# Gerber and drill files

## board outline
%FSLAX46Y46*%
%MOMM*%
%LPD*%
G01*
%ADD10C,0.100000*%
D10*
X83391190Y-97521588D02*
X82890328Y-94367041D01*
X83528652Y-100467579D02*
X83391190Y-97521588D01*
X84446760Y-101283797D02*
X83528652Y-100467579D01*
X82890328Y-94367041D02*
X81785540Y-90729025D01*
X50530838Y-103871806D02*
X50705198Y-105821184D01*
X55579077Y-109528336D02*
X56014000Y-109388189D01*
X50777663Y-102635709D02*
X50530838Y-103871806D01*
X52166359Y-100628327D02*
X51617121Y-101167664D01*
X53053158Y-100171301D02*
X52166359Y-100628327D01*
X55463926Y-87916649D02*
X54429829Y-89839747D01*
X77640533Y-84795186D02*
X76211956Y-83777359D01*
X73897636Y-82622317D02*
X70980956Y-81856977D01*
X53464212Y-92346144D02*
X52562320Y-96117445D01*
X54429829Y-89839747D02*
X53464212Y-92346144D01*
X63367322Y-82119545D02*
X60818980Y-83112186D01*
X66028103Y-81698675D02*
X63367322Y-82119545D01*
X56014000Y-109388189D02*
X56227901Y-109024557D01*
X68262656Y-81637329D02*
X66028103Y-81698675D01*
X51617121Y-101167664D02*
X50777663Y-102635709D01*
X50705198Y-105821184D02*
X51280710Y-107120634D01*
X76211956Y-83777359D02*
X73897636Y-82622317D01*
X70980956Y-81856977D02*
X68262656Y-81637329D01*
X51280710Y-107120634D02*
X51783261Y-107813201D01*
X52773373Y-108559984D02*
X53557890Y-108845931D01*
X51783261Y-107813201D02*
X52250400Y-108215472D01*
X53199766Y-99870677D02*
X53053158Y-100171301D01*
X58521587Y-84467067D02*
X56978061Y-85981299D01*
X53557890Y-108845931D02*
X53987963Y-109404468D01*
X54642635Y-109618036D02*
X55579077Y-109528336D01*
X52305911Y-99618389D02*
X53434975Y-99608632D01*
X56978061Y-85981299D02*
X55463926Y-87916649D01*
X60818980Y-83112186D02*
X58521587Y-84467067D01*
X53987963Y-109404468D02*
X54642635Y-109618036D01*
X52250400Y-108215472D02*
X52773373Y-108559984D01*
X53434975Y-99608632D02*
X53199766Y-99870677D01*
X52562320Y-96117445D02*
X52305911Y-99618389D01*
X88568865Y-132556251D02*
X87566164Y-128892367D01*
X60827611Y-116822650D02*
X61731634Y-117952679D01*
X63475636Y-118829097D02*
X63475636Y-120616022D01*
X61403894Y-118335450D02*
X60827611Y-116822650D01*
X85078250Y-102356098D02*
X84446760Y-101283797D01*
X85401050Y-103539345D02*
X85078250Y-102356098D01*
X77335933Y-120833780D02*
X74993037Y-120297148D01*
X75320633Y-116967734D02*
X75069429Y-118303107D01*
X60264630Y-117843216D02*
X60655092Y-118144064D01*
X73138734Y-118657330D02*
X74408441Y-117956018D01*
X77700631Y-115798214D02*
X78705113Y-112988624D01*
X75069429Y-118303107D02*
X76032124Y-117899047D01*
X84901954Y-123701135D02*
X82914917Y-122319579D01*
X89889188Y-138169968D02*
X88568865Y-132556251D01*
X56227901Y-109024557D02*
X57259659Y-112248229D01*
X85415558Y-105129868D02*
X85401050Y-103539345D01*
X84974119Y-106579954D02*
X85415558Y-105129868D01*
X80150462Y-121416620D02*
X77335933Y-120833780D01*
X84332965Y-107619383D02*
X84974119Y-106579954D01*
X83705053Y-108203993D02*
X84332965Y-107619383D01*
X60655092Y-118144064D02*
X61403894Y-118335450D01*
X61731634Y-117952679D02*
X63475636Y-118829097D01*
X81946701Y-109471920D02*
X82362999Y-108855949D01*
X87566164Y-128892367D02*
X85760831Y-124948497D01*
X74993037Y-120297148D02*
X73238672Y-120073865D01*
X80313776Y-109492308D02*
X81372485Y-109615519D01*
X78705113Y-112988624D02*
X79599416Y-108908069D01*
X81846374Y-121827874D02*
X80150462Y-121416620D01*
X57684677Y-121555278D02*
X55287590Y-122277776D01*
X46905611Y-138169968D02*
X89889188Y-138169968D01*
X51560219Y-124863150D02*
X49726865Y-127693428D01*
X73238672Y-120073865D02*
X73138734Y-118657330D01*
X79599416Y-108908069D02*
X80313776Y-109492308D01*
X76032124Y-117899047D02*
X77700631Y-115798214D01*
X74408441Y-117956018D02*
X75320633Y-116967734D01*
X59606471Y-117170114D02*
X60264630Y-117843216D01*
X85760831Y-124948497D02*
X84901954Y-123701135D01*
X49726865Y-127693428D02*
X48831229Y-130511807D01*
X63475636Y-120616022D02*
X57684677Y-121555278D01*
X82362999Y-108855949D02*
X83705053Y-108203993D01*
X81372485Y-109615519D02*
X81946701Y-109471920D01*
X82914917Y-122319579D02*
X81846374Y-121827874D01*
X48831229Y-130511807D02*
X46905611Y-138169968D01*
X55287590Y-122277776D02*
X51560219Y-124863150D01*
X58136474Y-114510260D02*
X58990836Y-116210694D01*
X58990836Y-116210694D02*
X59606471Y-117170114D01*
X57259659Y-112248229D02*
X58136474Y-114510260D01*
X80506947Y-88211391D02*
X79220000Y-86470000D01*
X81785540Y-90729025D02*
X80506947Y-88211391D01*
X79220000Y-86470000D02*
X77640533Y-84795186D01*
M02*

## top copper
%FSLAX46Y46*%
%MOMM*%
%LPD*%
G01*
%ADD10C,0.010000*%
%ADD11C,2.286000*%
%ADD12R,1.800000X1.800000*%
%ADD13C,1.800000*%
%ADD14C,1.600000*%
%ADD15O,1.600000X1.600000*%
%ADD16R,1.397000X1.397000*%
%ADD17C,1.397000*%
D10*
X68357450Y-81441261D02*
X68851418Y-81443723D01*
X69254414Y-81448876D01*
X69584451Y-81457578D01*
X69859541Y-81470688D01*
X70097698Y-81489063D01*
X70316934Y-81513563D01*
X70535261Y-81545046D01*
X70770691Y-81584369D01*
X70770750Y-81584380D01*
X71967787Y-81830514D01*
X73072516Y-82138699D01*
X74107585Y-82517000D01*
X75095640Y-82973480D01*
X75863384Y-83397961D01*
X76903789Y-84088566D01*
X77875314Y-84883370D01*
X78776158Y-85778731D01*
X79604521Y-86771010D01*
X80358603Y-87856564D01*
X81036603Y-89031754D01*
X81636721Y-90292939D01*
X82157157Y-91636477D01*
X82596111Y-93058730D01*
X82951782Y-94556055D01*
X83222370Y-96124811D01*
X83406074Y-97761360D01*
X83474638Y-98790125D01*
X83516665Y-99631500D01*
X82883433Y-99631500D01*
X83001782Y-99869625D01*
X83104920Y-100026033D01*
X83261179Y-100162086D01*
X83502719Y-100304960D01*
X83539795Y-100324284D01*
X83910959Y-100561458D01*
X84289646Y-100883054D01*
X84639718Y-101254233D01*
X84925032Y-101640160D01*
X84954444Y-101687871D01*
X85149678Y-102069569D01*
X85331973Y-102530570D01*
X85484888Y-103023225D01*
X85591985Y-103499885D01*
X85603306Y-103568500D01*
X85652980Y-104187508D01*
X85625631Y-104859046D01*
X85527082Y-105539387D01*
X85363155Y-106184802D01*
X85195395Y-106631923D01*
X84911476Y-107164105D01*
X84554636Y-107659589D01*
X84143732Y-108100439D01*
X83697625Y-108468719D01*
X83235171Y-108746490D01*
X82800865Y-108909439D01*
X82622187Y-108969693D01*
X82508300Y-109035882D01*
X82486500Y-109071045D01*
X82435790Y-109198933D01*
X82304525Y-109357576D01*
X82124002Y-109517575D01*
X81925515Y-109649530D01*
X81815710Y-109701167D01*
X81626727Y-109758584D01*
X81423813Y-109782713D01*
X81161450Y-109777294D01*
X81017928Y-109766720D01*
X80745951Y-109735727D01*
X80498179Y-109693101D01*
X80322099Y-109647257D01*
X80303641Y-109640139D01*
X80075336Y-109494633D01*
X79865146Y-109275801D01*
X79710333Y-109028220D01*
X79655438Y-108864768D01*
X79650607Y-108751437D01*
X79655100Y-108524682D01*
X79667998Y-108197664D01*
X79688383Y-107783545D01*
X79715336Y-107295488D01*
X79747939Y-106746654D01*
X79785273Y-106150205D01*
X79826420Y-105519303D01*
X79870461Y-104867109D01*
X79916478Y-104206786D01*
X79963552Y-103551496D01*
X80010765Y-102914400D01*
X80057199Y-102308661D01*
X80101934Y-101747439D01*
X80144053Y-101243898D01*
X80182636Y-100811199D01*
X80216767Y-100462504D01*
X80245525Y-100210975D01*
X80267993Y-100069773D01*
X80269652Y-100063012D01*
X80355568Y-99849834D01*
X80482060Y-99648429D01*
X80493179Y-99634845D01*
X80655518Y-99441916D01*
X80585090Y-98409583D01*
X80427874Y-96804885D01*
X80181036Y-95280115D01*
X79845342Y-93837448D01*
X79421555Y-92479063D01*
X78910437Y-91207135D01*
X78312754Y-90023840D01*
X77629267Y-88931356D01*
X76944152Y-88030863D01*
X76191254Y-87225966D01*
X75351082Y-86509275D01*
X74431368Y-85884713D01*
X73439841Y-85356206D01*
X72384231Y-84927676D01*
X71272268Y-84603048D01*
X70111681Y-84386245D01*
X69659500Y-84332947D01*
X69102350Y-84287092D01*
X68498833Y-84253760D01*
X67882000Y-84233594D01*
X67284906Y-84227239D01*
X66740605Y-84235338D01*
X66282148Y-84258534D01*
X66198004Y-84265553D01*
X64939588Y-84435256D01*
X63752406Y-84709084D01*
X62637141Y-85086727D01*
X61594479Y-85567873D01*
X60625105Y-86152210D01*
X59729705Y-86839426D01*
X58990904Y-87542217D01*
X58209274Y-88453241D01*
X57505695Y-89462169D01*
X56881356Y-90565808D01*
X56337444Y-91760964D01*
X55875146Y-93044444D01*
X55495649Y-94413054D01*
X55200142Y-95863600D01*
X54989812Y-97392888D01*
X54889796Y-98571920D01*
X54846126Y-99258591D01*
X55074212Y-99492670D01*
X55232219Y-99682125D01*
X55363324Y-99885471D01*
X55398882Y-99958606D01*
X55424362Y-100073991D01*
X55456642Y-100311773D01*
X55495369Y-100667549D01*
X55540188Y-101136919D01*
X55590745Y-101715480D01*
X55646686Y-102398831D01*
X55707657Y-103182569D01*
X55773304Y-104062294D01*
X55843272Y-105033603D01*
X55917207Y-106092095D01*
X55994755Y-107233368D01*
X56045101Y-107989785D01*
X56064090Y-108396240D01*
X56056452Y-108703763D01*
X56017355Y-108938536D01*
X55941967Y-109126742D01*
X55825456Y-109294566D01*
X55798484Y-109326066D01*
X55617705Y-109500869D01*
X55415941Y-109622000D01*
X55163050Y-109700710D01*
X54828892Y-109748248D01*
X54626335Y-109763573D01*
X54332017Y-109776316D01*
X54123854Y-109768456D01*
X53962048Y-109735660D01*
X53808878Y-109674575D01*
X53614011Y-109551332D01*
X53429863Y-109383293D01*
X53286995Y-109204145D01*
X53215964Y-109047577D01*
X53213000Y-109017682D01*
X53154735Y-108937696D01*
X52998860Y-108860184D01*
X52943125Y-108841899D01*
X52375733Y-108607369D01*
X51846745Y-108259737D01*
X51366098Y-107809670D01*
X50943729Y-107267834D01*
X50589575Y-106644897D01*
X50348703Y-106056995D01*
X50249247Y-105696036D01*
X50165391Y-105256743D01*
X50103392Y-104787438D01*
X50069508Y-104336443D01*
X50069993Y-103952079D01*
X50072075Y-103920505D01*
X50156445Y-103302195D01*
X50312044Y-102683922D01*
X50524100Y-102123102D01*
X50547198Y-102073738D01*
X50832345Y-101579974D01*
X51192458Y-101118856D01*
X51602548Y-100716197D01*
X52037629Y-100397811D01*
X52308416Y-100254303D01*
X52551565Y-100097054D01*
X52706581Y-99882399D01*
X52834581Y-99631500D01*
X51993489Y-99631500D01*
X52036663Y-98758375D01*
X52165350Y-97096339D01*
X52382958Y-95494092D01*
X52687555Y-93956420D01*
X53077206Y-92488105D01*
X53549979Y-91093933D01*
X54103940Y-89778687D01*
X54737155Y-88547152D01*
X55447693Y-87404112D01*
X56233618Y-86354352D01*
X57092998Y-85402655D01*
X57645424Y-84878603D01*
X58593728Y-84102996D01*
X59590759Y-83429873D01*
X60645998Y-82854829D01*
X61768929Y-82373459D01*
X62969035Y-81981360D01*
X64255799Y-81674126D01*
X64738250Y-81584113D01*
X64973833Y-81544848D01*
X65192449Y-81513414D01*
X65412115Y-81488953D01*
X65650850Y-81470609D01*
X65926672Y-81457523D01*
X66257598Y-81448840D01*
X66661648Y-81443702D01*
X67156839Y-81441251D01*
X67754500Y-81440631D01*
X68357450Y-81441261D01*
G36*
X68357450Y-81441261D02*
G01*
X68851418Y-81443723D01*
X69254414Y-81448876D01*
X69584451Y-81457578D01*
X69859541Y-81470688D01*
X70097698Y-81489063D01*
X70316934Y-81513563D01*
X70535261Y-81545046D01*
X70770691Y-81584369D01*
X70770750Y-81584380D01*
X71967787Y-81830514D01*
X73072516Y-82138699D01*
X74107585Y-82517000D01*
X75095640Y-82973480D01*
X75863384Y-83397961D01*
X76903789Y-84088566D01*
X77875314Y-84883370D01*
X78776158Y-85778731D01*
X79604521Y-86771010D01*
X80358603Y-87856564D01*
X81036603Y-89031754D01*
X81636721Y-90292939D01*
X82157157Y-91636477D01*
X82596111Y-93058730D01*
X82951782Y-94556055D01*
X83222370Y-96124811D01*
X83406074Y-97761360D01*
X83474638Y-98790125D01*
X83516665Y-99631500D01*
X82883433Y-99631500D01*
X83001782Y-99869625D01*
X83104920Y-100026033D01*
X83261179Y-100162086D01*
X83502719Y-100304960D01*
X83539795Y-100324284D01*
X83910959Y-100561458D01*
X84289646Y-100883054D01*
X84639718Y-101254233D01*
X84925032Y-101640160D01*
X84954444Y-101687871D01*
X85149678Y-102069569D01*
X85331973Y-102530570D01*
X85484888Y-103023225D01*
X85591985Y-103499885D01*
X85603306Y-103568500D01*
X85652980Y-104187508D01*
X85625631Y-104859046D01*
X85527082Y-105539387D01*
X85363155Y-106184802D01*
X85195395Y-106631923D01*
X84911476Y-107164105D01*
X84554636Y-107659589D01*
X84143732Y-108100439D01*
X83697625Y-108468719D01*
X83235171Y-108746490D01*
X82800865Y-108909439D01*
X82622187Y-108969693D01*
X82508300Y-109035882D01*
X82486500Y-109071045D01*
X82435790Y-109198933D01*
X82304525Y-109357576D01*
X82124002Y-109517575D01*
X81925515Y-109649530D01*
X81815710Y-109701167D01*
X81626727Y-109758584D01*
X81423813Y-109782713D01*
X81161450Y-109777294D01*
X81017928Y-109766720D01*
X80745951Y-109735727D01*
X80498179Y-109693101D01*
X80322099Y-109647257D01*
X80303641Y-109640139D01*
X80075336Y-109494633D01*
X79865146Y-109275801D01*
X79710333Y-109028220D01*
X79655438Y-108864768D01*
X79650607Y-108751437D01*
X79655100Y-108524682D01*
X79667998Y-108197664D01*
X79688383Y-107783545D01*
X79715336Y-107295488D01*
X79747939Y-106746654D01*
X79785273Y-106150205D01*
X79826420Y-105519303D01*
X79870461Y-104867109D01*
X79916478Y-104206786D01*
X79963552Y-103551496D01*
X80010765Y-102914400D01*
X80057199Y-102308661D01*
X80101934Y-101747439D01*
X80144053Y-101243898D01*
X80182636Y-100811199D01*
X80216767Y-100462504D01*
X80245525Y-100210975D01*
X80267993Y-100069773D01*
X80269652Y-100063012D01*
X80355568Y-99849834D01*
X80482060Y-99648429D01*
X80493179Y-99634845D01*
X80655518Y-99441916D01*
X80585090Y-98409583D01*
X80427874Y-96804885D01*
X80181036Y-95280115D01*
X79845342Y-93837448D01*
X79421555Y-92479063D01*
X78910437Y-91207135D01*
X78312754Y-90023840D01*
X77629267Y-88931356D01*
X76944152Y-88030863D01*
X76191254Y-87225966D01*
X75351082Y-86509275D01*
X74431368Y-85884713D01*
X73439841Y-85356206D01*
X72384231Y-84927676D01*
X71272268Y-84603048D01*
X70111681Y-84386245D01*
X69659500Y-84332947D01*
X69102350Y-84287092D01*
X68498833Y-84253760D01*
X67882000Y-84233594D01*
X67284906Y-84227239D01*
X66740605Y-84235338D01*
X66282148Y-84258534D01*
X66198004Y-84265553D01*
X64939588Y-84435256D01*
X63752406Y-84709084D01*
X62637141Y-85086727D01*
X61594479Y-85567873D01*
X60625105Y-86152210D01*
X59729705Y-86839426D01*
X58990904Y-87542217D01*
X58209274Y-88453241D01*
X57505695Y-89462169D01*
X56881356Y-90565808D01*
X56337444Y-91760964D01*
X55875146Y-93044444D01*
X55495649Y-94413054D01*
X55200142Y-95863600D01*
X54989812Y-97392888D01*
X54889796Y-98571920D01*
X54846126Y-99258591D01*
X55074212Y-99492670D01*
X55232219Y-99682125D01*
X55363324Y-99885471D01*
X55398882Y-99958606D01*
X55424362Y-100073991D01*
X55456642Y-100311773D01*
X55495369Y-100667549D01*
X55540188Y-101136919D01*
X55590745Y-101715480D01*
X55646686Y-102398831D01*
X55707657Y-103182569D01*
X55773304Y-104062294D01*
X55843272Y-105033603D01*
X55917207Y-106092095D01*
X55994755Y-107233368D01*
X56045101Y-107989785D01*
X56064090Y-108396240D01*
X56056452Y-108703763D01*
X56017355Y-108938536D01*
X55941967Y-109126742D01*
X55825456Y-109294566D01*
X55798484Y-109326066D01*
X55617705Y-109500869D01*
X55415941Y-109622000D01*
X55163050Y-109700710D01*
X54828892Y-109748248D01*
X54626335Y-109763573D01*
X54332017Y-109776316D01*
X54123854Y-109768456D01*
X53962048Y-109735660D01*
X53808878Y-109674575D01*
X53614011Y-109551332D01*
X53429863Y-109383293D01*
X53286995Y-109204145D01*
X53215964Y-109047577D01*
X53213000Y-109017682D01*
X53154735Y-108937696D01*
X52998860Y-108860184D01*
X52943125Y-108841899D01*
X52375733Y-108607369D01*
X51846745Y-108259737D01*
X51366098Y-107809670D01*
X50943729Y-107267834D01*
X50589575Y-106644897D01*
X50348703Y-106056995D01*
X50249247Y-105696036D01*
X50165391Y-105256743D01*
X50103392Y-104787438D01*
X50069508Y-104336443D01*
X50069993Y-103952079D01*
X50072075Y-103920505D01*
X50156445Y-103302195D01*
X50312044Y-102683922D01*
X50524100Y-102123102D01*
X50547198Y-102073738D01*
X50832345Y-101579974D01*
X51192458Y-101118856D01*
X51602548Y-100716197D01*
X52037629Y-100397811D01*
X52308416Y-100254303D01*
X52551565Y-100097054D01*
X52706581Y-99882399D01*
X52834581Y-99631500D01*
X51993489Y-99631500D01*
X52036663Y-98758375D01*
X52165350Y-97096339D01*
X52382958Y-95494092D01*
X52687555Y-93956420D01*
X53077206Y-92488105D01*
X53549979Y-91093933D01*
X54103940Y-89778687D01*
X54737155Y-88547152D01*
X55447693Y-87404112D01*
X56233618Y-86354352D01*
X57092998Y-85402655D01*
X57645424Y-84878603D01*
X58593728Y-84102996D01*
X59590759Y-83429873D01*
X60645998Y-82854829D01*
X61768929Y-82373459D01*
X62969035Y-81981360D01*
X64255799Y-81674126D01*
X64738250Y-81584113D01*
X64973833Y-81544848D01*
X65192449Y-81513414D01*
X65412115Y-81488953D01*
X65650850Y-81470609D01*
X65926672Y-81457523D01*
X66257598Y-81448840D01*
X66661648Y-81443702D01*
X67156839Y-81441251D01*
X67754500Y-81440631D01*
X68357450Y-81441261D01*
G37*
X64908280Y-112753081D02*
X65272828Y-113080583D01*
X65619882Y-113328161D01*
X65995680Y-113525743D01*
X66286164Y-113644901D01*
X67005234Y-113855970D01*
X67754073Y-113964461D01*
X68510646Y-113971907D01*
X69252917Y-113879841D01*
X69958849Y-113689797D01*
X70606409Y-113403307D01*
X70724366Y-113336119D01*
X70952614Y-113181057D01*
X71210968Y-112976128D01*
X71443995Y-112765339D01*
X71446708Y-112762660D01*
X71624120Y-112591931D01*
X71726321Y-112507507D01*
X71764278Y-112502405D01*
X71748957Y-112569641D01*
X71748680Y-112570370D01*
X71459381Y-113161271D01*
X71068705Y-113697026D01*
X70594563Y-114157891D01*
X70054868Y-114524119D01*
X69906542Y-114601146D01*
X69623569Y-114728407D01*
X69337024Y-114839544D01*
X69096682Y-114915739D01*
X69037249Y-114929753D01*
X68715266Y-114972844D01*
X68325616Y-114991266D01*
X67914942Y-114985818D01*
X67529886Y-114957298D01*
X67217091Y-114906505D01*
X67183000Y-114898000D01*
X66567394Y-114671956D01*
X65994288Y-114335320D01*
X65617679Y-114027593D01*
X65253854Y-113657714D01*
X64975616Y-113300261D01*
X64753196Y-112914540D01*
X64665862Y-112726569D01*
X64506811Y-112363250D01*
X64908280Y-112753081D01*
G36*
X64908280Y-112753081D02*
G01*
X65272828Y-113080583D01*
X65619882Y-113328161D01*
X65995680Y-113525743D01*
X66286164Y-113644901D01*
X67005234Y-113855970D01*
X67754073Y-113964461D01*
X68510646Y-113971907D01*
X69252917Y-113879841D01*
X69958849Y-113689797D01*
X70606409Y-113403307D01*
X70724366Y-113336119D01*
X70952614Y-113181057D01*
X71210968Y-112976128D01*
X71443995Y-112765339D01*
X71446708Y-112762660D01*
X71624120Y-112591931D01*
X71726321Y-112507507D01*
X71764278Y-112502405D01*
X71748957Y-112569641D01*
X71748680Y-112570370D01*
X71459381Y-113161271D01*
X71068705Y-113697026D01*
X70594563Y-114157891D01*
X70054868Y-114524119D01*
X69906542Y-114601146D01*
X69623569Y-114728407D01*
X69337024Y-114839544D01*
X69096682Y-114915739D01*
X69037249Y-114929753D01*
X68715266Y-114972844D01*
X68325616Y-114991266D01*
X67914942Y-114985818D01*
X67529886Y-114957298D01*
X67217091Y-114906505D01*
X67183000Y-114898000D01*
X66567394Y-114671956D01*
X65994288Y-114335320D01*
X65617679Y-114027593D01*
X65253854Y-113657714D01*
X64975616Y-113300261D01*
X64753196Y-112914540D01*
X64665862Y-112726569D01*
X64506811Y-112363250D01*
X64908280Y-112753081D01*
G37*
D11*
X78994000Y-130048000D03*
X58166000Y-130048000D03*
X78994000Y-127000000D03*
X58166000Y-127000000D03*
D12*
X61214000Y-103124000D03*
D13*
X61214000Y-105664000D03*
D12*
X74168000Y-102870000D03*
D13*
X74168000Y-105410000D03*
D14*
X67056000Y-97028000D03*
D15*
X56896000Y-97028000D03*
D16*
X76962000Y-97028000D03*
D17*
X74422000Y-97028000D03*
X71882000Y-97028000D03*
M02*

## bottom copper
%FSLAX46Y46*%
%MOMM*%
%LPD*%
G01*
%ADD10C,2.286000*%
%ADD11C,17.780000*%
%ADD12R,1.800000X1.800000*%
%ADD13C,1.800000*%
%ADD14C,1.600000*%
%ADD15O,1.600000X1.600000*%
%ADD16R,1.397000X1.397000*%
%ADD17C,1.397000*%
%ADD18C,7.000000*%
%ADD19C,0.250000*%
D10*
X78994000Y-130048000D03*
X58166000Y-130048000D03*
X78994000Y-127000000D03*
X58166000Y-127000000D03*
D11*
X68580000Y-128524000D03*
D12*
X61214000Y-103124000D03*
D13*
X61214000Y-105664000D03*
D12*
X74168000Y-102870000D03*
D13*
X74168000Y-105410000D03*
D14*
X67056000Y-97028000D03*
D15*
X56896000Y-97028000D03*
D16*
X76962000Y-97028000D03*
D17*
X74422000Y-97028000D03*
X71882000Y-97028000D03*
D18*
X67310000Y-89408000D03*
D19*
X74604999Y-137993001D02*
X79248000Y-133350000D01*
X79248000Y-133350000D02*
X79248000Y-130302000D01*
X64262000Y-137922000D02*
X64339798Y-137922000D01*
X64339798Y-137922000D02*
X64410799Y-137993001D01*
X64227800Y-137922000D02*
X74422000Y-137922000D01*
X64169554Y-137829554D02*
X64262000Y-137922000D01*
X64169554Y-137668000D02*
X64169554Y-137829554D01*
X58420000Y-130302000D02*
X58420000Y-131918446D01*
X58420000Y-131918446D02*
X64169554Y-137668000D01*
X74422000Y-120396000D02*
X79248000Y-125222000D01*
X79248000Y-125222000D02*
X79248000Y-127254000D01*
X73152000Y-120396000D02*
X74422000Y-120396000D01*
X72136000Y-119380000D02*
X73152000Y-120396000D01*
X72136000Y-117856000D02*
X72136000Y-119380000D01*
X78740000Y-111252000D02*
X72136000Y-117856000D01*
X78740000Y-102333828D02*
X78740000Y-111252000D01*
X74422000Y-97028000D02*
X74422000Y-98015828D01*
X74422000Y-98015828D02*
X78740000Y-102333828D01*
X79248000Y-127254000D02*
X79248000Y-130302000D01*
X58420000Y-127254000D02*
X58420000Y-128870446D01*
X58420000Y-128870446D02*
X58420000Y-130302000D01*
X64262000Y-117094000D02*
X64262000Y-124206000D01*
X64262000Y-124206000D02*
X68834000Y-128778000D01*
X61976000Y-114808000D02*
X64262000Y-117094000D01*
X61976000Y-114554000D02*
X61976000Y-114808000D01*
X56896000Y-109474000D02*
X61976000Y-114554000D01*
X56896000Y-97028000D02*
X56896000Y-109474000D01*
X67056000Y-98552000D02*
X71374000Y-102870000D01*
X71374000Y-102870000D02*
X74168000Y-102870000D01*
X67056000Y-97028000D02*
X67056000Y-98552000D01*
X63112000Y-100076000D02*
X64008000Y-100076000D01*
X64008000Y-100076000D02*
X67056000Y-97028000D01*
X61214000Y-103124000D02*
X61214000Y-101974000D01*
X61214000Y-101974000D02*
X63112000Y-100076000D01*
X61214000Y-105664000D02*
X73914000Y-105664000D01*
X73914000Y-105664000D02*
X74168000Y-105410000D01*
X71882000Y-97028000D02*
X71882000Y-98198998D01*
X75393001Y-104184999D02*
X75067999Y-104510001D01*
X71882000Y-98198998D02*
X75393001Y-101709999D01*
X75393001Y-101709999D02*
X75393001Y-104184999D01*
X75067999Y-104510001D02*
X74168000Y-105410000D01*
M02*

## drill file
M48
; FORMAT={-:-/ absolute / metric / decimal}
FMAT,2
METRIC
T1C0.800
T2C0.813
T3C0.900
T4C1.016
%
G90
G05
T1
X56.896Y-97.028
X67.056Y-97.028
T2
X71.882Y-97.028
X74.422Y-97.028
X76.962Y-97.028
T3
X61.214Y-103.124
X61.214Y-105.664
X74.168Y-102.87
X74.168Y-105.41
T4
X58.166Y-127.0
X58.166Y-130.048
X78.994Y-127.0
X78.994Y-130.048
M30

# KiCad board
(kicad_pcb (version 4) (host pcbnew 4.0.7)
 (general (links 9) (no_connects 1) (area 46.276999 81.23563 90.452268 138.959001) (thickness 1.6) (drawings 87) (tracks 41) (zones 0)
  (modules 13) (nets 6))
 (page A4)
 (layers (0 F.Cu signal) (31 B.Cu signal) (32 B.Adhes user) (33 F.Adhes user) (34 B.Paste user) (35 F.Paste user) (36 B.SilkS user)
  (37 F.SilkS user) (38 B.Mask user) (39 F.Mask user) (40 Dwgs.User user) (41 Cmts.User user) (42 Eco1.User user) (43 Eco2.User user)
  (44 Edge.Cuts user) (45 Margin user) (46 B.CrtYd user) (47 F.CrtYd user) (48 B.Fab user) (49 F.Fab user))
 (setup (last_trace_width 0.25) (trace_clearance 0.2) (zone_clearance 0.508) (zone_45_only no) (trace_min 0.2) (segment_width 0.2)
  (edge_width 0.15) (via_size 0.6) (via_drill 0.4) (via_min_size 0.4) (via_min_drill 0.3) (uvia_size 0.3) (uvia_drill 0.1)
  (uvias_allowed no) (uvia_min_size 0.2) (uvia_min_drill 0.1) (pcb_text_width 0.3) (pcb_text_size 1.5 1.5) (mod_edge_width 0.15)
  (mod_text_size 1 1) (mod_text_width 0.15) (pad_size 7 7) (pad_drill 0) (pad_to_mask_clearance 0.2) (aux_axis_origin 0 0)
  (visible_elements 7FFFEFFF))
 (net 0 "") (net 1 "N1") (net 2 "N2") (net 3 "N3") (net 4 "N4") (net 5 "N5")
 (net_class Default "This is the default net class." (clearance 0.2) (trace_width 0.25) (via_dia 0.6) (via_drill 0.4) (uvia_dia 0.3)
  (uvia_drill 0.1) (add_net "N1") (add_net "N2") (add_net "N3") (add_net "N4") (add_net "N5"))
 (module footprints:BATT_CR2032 (layer B.Cu) (at 68.58 128.524 180)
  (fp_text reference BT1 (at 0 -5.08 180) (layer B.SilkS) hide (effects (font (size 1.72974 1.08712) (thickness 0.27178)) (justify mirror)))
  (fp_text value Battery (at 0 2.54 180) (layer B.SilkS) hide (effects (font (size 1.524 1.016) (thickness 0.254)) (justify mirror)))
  (pad 1 thru_hole circle (at -10.414 -1.524 180) (size 2.286 2.286) (drill 1.016) (layers *.Cu *.Mask B.SilkS) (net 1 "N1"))
  (pad 1 thru_hole circle (at 10.414 -1.524 180) (size 2.286 2.286) (drill 1.016) (layers *.Cu *.Mask B.SilkS) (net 1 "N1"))
  (pad 1 thru_hole circle (at -10.414 1.524 180) (size 2.286 2.286) (drill 1.016) (layers *.Cu *.Mask B.SilkS) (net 1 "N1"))
  (pad 1 thru_hole circle (at 10.414 1.524 180) (size 2.286 2.286) (drill 1.016) (layers *.Cu *.Mask B.SilkS) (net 1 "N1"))
  (pad 2 smd circle (at 0 0 180) (size 17.78 17.78) (layers B.Cu B.Paste B.Mask) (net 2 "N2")))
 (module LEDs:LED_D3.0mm (layer F.Cu) (at 61.214 103.124 270)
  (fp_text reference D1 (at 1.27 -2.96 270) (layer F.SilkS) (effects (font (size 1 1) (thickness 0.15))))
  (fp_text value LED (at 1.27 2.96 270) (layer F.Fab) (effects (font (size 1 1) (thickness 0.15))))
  (pad 1 thru_hole rect (at 0 0 270) (size 1.8 1.8) (drill 0.9) (layers *.Cu *.Mask) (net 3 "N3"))
  (pad 2 thru_hole circle (at 2.54 0 270) (size 1.8 1.8) (drill 0.9) (layers *.Cu *.Mask) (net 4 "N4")))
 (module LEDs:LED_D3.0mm (layer F.Cu) (at 74.168 102.87 270)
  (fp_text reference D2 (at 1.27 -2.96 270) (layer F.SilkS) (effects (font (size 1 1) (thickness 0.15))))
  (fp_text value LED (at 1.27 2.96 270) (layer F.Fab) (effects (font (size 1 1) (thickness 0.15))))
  (pad 1 thru_hole rect (at 0 0 270) (size 1.8 1.8) (drill 0.9) (layers *.Cu *.Mask) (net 3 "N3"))
  (pad 2 thru_hole circle (at 2.54 0 270) (size 1.8 1.8) (drill 0.9) (layers *.Cu *.Mask) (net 4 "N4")))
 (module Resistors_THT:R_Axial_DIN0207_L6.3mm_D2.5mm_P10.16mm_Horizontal (layer B.Cu) (at 67.056 97.028 180)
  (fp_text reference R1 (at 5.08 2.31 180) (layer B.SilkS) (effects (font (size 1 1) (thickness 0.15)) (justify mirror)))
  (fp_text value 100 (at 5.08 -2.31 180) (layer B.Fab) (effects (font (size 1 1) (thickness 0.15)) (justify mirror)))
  (pad 1 thru_hole circle (at 0 0 180) (size 1.6 1.6) (drill 0.8) (layers *.Cu *.Mask) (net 3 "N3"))
  (pad 2 thru_hole oval (at 10.16 0 180) (size 1.6 1.6) (drill 0.8) (layers *.Cu *.Mask) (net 2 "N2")))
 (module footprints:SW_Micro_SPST (layer B.Cu) (at 74.422 97.028 180)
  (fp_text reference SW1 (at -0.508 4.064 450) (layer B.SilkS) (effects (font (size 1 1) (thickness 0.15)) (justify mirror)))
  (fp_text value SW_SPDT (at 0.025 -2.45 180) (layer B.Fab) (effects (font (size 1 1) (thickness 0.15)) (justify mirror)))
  (pad 1 thru_hole rect (at -2.54 0 180) (size 1.397 1.397) (drill 0.8128) (layers *.Cu *.Mask B.SilkS) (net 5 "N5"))
  (pad 2 thru_hole circle (at 0 0 180) (size 1.397 1.397) (drill 0.8128) (layers *.Cu *.Mask B.SilkS) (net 1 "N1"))
  (pad 3 thru_hole circle (at 2.54 0 180) (size 1.397 1.397) (drill 0.8128) (layers *.Cu *.Mask B.SilkS) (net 4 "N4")))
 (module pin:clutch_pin (layer F.Cu) (at 67.31 89.408)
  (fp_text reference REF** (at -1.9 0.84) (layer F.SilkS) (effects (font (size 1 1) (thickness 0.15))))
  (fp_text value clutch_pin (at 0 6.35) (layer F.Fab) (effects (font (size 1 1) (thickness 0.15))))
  (pad 1 smd circle (at 0 0 90) (size 7 7) (layers B.Cu B.Paste B.SilkS B.Mask)))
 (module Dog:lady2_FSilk (layer F.Cu) (at 68.326 109.728)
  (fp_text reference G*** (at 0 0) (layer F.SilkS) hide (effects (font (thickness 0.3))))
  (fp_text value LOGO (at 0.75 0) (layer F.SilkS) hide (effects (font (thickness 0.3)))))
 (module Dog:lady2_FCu (layer F.Cu) (at 67.818 97.536)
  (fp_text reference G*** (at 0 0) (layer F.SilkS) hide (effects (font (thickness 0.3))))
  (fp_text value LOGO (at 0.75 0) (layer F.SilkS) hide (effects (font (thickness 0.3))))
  (fp_poly
   (pts (xy 0.53945 -16.094739) (xy 1.033418 -16.092277) (xy 1.436414 -16.087124) (xy 1.766451 -16.078422) (xy 2.041541 -16.065312)
    (xy 2.279698 -16.046937) (xy 2.498934 -16.022437) (xy 2.717261 -15.990954) (xy 2.952691 -15.951631) (xy 2.95275 -15.95162)
    (xy 4.149787 -15.705486) (xy 5.254516 -15.397301) (xy 6.289585 -15.019) (xy 7.27764 -14.56252) (xy 8.045384 -14.138039)
    (xy 9.085789 -13.447434) (xy 10.057314 -12.65263) (xy 10.958158 -11.757269) (xy 11.786521 -10.76499) (xy 12.540603 -9.679436)
    (xy 13.218603 -8.504246) (xy 13.818721 -7.243061) (xy 14.339157 -5.899523) (xy 14.778111 -4.47727) (xy 15.133782 -2.979945)
    (xy 15.40437 -1.411189) (xy 15.588074 0.22536) (xy 15.656638 1.254125) (xy 15.698665 2.0955) (xy 15.065433 2.0955)
    (xy 15.183782 2.333625) (xy 15.28692 2.490033) (xy 15.443179 2.626086) (xy 15.684719 2.76896) (xy 15.721795 2.788284)
    (xy 16.092959 3.025458) (xy 16.471646 3.347054) (xy 16.821718 3.718233) (xy 17.107032 4.10416) (xy 17.136444 4.151871)
    (xy 17.331678 4.533569) (xy 17.513973 4.99457) (xy 17.666888 5.487225) (xy 17.773985 5.963885) (xy 17.785306 6.0325)
    (xy 17.83498 6.651508) (xy 17.807631 7.323046) (xy 17.709082 8.003387) (xy 17.545155 8.648802) (xy 17.377395 9.095923)
    (xy 17.093476 9.628105) (xy 16.736636 10.123589) (xy 16.325732 10.564439) (xy 15.879625 10.932719) (xy 15.417171 11.21049)
    (xy 14.982865 11.373439) (xy 14.804187 11.433693) (xy 14.6903 11.499882) (xy 14.6685 11.535045) (xy 14.61779 11.662933)
    (xy 14.486525 11.821576) (xy 14.306002 11.981575) (xy 14.107515 12.11353) (xy 13.99771 12.165167) (xy 13.808727 12.222584)
    (xy 13.605813 12.246713) (xy 13.34345 12.241294) (xy 13.199928 12.23072) (xy 12.927951 12.199727) (xy 12.680179 12.157101)
    (xy 12.504099 12.111257) (xy 12.485641 12.104139) (xy 12.257336 11.958633) (xy 12.047146 11.739801) (xy 11.892333 11.49222)
    (xy 11.837438 11.328768) (xy 11.832607 11.215437) (xy 11.8371 10.988682) (xy 11.849998 10.661664) (xy 11.870383 10.247545)
    (xy 11.897336 9.759488) (xy 11.929939 9.210654) (xy 11.967273 8.614205) (xy 12.00842 7.983303) (xy 12.052461 7.331109)
    (xy 12.098478 6.670786) (xy 12.145552 6.015496) (xy 12.192765 5.3784) (xy 12.239199 4.772661) (xy 12.283934 4.211439)
    (xy 12.326053 3.707898) (xy 12.364636 3.275199) (xy 12.398767 2.926504) (xy 12.427525 2.674975) (xy 12.449993 2.533773)
    (xy 12.451652 2.527012) (xy 12.537568 2.313834) (xy 12.66406 2.112429) (xy 12.675179 2.098845) (xy 12.837518 1.905916)
    (xy 12.76709 0.873583) (xy 12.609874 -0.731115) (xy 12.363036 -2.255885) (xy 12.027342 -3.698552) (xy 11.603555 -5.056937)
    (xy 11.092437 -6.328865) (xy 10.494754 -7.51216) (xy 9.811267 -8.604644) (xy 9.126152 -9.505137) (xy 8.373254 -10.310034)
    (xy 7.533082 -11.026725) (xy 6.613368 -11.651287) (xy 5.621841 -12.179794) (xy 4.566231 -12.608324) (xy 3.454268 -12.932952)
    (xy 2.293681 -13.149755) (xy 1.8415 -13.203053) (xy 1.28435 -13.248908) (xy 0.680833 -13.28224) (xy 0.064 -13.302406)
    (xy -0.533094 -13.308761) (xy -1.077395 -13.300662) (xy -1.535852 -13.277466) (xy -1.619996 -13.270447) (xy -2.878412 -13.100744)
    (xy -4.065594 -12.826916) (xy -5.180859 -12.449273) (xy -6.223521 -11.968127) (xy -7.192895 -11.38379) (xy -8.088295 -10.696574)
    (xy -8.827096 -9.993783) (xy -9.608726 -9.082759) (xy -10.312305 -8.073831) (xy -10.936644 -6.970192) (xy -11.480556 -5.775036)
    (xy -11.942854 -4.491556) (xy -12.322351 -3.122946) (xy -12.617858 -1.6724) (xy -12.828188 -0.143112) (xy -12.928204 1.03592)
    (xy -12.971874 1.722591) (xy -12.743788 1.95667) (xy -12.585781 2.146125) (xy -12.454676 2.349471) (xy -12.419118 2.422606)
    (xy -12.393638 2.537991) (xy -12.361358 2.775773) (xy -12.322631 3.131549) (xy -12.277812 3.600919) (xy -12.227255 4.17948)
    (xy -12.171314 4.862831) (xy -12.110343 5.646569) (xy -12.044696 6.526294) (xy -11.974728 7.497603) (xy -11.900793 8.556095)
    (xy -11.823245 9.697368) (xy -11.772899 10.453785) (xy -11.75391 10.86024) (xy -11.761548 11.167763) (xy -11.800645 11.402536)
    (xy -11.876033 11.590742) (xy -11.992544 11.758566) (xy -12.019516 11.790066) (xy -12.200295 11.964869) (xy -12.402059 12.086)
    (xy -12.65495 12.16471) (xy -12.989108 12.212248) (xy -13.191665 12.227573) (xy -13.485983 12.240316) (xy -13.694146 12.232456)
    (xy -13.855952 12.19966) (xy -14.009122 12.138575) (xy -14.203989 12.015332) (xy -14.388137 11.847293) (xy -14.531005 11.668145)
    (xy -14.602036 11.511577) (xy -14.605 11.481682) (xy -14.663265 11.401696) (xy -14.81914 11.324184) (xy -14.874875 11.305899)
    (xy -15.442267 11.071369) (xy -15.971255 10.723737) (xy -16.451902 10.27367) (xy -16.874271 9.731834) (xy -17.228425 9.108897)
    (xy -17.469297 8.520995) (xy -17.568753 8.160036) (xy -17.652609 7.720743) (xy -17.714608 7.251438) (xy -17.748492 6.800443)
    (xy -17.748007 6.416079) (xy -17.745925 6.384505) (xy -17.661555 5.766195) (xy -17.505956 5.147922) (xy -17.2939 4.587102)
    (xy -17.270802 4.537738) (xy -16.985655 4.043974) (xy -16.625542 3.582856) (xy -16.215452 3.180197) (xy -15.780371 2.861811)
    (xy -15.509584 2.718303) (xy -15.266435 2.561054) (xy -15.111419 2.346399) (xy -14.983419 2.0955) (xy -15.824511 2.0955)
    (xy -15.781337 1.222375) (xy -15.65265 -0.439661) (xy -15.435042 -2.041908) (xy -15.130445 -3.57958) (xy -14.740794 -5.047895)
    (xy -14.268021 -6.442067) (xy -13.71406 -7.757313) (xy -13.080845 -8.988848) (xy -12.370307 -10.131888) (xy -11.584382 -11.181648)
    (xy -10.725002 -12.133345) (xy -10.172576 -12.657397) (xy -9.224272 -13.433004) (xy -8.227241 -14.106127) (xy -7.172002 -14.681171)
    (xy -6.049071 -15.162541) (xy -4.848965 -15.55464) (xy -3.562201 -15.861874) (xy -3.07975 -15.951887) (xy -2.844167 -15.991152)
    (xy -2.625551 -16.022586) (xy -2.405885 -16.047047) (xy -2.16715 -16.065391) (xy -1.891328 -16.078477) (xy -1.560402 -16.08716)
    (xy -1.156352 -16.092298) (xy -0.661161 -16.094749) (xy -0.0635 -16.095369) (xy 0.53945 -16.094739))
   (layer F.Cu) (width 0.01)))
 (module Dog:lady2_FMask (layer F.Cu) (at 67.818 97.536)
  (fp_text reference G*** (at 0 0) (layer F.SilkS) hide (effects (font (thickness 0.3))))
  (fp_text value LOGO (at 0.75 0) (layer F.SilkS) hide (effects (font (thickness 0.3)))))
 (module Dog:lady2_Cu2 (layer F.Cu) (at 68.326 98.806)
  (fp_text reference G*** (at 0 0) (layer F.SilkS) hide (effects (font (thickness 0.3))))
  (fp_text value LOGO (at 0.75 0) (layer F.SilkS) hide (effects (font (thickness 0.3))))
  (fp_poly
   (pts (xy -3.41772 13.947081) (xy -3.053172 14.274583) (xy -2.706118 14.522161) (xy -2.33032 14.719743) (xy -2.039836 14.838901)
    (xy -1.320766 15.04997) (xy -0.571927 15.158461) (xy 0.184646 15.165907) (xy 0.926917 15.073841) (xy 1.632849 14.883797)
    (xy 2.280409 14.597307) (xy 2.398366 14.530119) (xy 2.626614 14.375057) (xy 2.884968 14.170128) (xy 3.117995 13.959339)
    (xy 3.120708 13.95666) (xy 3.29812 13.785931) (xy 3.400321 13.701507) (xy 3.438278 13.696405) (xy 3.422957 13.763641)
    (xy 3.42268 13.76437) (xy 3.133381 14.355271) (xy 2.742705 14.891026) (xy 2.268563 15.351891) (xy 1.728868 15.718119)
    (xy 1.580542 15.795146) (xy 1.297569 15.922407) (xy 1.011024 16.033544) (xy 0.770682 16.109739) (xy 0.711249 16.123753)
    (xy 0.389266 16.166844) (xy -0.000384 16.185266) (xy -0.411058 16.179818) (xy -0.796114 16.151298) (xy -1.108909 16.100505)
    (xy -1.143 16.092) (xy -1.758606 15.865956) (xy -2.331712 15.52932) (xy -2.708321 15.221593) (xy -3.072146 14.851714)
    (xy -3.350384 14.494261) (xy -3.572804 14.10854) (xy -3.660138 13.920569) (xy -3.819189 13.55725) (xy -3.41772 13.947081))
   (layer F.Cu) (width 0.01)))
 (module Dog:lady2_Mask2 (layer F.Cu) (at 68.326 98.806)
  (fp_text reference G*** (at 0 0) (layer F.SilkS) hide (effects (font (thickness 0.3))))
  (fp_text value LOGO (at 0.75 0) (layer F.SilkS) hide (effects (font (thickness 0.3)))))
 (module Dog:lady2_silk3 (layer F.Cu) (at 68.326 106.68)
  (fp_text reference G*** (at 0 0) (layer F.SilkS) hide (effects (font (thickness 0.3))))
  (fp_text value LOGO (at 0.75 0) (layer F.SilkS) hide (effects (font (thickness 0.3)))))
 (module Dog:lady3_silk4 (layer F.Cu) (at 68.58 111.76)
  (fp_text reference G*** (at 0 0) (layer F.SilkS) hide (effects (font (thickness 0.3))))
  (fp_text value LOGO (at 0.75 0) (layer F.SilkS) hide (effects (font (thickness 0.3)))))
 (gr_line (start 83.39119 97.521588) (end 82.890328 94.367041) (layer Edge.Cuts) (width 0.1))
 (gr_line (start 83.528652 100.467579) (end 83.39119 97.521588) (layer Edge.Cuts) (width 0.1))
 (gr_line (start 84.44676 101.283797) (end 83.528652 100.467579) (layer Edge.Cuts) (width 0.1))
 (gr_line (start 82.890328 94.367041) (end 81.78554 90.729025) (layer Edge.Cuts) (width 0.1))
 (gr_line (start 50.530838 103.871806) (end 50.705198 105.821184) (layer Edge.Cuts) (width 0.1))
 (gr_line (start 55.579077 109.528336) (end 56.014 109.388189) (layer Edge.Cuts) (width 0.1))
 (gr_line (start 50.777663 102.635709) (end 50.530838 103.871806) (layer Edge.Cuts) (width 0.1))
 (gr_line (start 52.166359 100.628327) (end 51.617121 101.167664) (layer Edge.Cuts) (width 0.1))
 (gr_line (start 53.053158 100.171301) (end 52.166359 100.628327) (layer Edge.Cuts) (width 0.1))
 (gr_line (start 55.463926 87.916649) (end 54.429829 89.839747) (layer Edge.Cuts) (width 0.1))
 (gr_line (start 77.640533 84.795186) (end 76.211956 83.777359) (layer Edge.Cuts) (width 0.1))
 (gr_line (start 73.897636 82.622317) (end 70.980956 81.856977) (layer Edge.Cuts) (width 0.1))
 (gr_line (start 53.464212 92.346144) (end 52.56232 96.117445) (layer Edge.Cuts) (width 0.1))
 (gr_line (start 54.429829 89.839747) (end 53.464212 92.346144) (layer Edge.Cuts) (width 0.1))
 (gr_line (start 63.367322 82.119545) (end 60.81898 83.112186) (layer Edge.Cuts) (width 0.1))
 (gr_line (start 66.028103 81.698675) (end 63.367322 82.119545) (layer Edge.Cuts) (width 0.1))
 (gr_line (start 56.014 109.388189) (end 56.227901 109.024557) (layer Edge.Cuts) (width 0.1))
 (gr_line (start 68.262656 81.637329) (end 66.028103 81.698675) (layer Edge.Cuts) (width 0.1))
 (gr_line (start 51.617121 101.167664) (end 50.777663 102.635709) (layer Edge.Cuts) (width 0.1))
 (gr_line (start 50.705198 105.821184) (end 51.28071 107.120634) (layer Edge.Cuts) (width 0.1))
 (gr_line (start 76.211956 83.777359) (end 73.897636 82.622317) (layer Edge.Cuts) (width 0.1))
 (gr_line (start 70.980956 81.856977) (end 68.262656 81.637329) (layer Edge.Cuts) (width 0.1))
 (gr_line (start 51.28071 107.120634) (end 51.783261 107.813201) (layer Edge.Cuts) (width 0.1))
 (gr_line (start 52.773373 108.559984) (end 53.55789 108.845931) (layer Edge.Cuts) (width 0.1))
 (gr_line (start 51.783261 107.813201) (end 52.2504 108.215472) (layer Edge.Cuts) (width 0.1))
 (gr_line (start 53.199766 99.870677) (end 53.053158 100.171301) (layer Edge.Cuts) (width 0.1))
 (gr_line (start 58.521587 84.467067) (end 56.978061 85.981299) (layer Edge.Cuts) (width 0.1))
 (gr_line (start 53.55789 108.845931) (end 53.987963 109.404468) (layer Edge.Cuts) (width 0.1))
 (gr_line (start 54.642635 109.618036) (end 55.579077 109.528336) (layer Edge.Cuts) (width 0.1))
 (gr_line (start 52.305911 99.618389) (end 53.434975 99.608632) (layer Edge.Cuts) (width 0.1))
 (gr_line (start 56.978061 85.981299) (end 55.463926 87.916649) (layer Edge.Cuts) (width 0.1))
 (gr_line (start 60.81898 83.112186) (end 58.521587 84.467067) (layer Edge.Cuts) (width 0.1))
 (gr_line (start 53.987963 109.404468) (end 54.642635 109.618036) (layer Edge.Cuts) (width 0.1))
 (gr_line (start 52.2504 108.215472) (end 52.773373 108.559984) (layer Edge.Cuts) (width 0.1))
 (gr_line (start 53.434975 99.608632) (end 53.199766 99.870677) (layer Edge.Cuts) (width 0.1))
 (gr_line (start 52.56232 96.117445) (end 52.305911 99.618389) (layer Edge.Cuts) (width 0.1))
 (gr_line (start 88.568865 132.556251) (end 87.566164 128.892367) (layer Edge.Cuts) (width 0.1))
 (gr_line (start 60.827611 116.82265) (end 61.731634 117.952679) (layer Edge.Cuts) (width 0.1))
 (gr_line (start 63.475636 118.829097) (end 63.475636 120.616022) (layer Edge.Cuts) (width 0.1))
 (gr_line (start 61.403894 118.33545) (end 60.827611 116.82265) (layer Edge.Cuts) (width 0.1))
 (gr_line (start 85.07825 102.356098) (end 84.44676 101.283797) (layer Edge.Cuts) (width 0.1))
 (gr_line (start 85.40105 103.539345) (end 85.07825 102.356098) (layer Edge.Cuts) (width 0.1))
 (gr_line (start 77.335933 120.83378) (end 74.993037 120.297148) (layer Edge.Cuts) (width 0.1))
 (gr_line (start 75.320633 116.967734) (end 75.069429 118.303107) (layer Edge.Cuts) (width 0.1))
 (gr_line (start 60.26463 117.843216) (end 60.655092 118.144064) (layer Edge.Cuts) (width 0.1))
 (gr_line (start 73.138734 118.65733) (end 74.408441 117.956018) (layer Edge.Cuts) (width 0.1))
 (gr_line (start 77.700631 115.798214) (end 78.705113 112.988624) (layer Edge.Cuts) (width 0.1))
 (gr_line (start 75.069429 118.303107) (end 76.032124 117.899047) (layer Edge.Cuts) (width 0.1))
 (gr_line (start 84.901954 123.701135) (end 82.914917 122.319579) (layer Edge.Cuts) (width 0.1))
 (gr_line (start 89.889188 138.169968) (end 88.568865 132.556251) (layer Edge.Cuts) (width 0.1))
 (gr_line (start 56.227901 109.024557) (end 57.259659 112.248229) (layer Edge.Cuts) (width 0.1))
 (gr_line (start 85.415558 105.129868) (end 85.40105 103.539345) (layer Edge.Cuts) (width 0.1))
 (gr_line (start 84.974119 106.579954) (end 85.415558 105.129868) (layer Edge.Cuts) (width 0.1))
 (gr_line (start 80.150462 121.41662) (end 77.335933 120.83378) (layer Edge.Cuts) (width 0.1))
 (gr_line (start 84.332965 107.619383) (end 84.974119 106.579954) (layer Edge.Cuts) (width 0.1))
 (gr_line (start 83.705053 108.203993) (end 84.332965 107.619383) (layer Edge.Cuts) (width 0.1))
 (gr_line (start 60.655092 118.144064) (end 61.403894 118.33545) (layer Edge.Cuts) (width 0.1))
 (gr_line (start 61.731634 117.952679) (end 63.475636 118.829097) (layer Edge.Cuts) (width 0.1))
 (gr_line (start 81.946701 109.47192) (end 82.362999 108.855949) (layer Edge.Cuts) (width 0.1))
 (gr_line (start 87.566164 128.892367) (end 85.760831 124.948497) (layer Edge.Cuts) (width 0.1))
 (gr_line (start 74.993037 120.297148) (end 73.238672 120.073865) (layer Edge.Cuts) (width 0.1))
 (gr_line (start 80.313776 109.492308) (end 81.372485 109.615519) (layer Edge.Cuts) (width 0.1))
 (gr_line (start 78.705113 112.988624) (end 79.599416 108.908069) (layer Edge.Cuts) (width 0.1))
 (gr_line (start 81.846374 121.827874) (end 80.150462 121.41662) (layer Edge.Cuts) (width 0.1))
 (gr_line (start 57.684677 121.555278) (end 55.28759 122.277776) (layer Edge.Cuts) (width 0.1))
 (gr_line (start 46.905611 138.169968) (end 89.889188 138.169968) (layer Edge.Cuts) (width 0.1))
 (gr_line (start 51.560219 124.86315) (end 49.726865 127.693428) (layer Edge.Cuts) (width 0.1))
 (gr_line (start 73.238672 120.073865) (end 73.138734 118.65733) (layer Edge.Cuts) (width 0.1))
 (gr_line (start 79.599416 108.908069) (end 80.313776 109.492308) (layer Edge.Cuts) (width 0.1))
 (gr_line (start 76.032124 117.899047) (end 77.700631 115.798214) (layer Edge.Cuts) (width 0.1))
 (gr_line (start 74.408441 117.956018) (end 75.320633 116.967734) (layer Edge.Cuts) (width 0.1))
 (gr_line (start 59.606471 117.170114) (end 60.26463 117.843216) (layer Edge.Cuts) (width 0.1))
 (gr_line (start 85.760831 124.948497) (end 84.901954 123.701135) (layer Edge.Cuts) (width 0.1))
 (gr_line (start 49.726865 127.693428) (end 48.831229 130.511807) (layer Edge.Cuts) (width 0.1))
 (gr_line (start 63.475636 120.616022) (end 57.684677 121.555278) (layer Edge.Cuts) (width 0.1))
 (gr_line (start 82.362999 108.855949) (end 83.705053 108.203993) (layer Edge.Cuts) (width 0.1))
 (gr_line (start 81.372485 109.615519) (end 81.946701 109.47192) (layer Edge.Cuts) (width 0.1))
 (gr_line (start 82.914917 122.319579) (end 81.846374 121.827874) (layer Edge.Cuts) (width 0.1))
 (gr_line (start 48.831229 130.511807) (end 46.905611 138.169968) (layer Edge.Cuts) (width 0.1))
 (gr_line (start 55.28759 122.277776) (end 51.560219 124.86315) (layer Edge.Cuts) (width 0.1))
 (gr_line (start 58.136474 114.51026) (end 58.990836 116.210694) (layer Edge.Cuts) (width 0.1))
 (gr_line (start 58.990836 116.210694) (end 59.606471 117.170114) (layer Edge.Cuts) (width 0.1))
 (gr_line (start 57.259659 112.248229) (end 58.136474 114.51026) (layer Edge.Cuts) (width 0.1))
 (gr_line (start 80.506947 88.211391) (end 79.22 86.47) (layer Edge.Cuts) (width 0.1))
 (gr_line (start 81.78554 90.729025) (end 80.506947 88.211391) (layer Edge.Cuts) (width 0.1))
 (gr_line (start 79.22 86.47) (end 77.640533 84.795186) (layer Edge.Cuts) (width 0.1))
 (segment (start 74.604999 137.993001) (end 79.248 133.35) (width 0.25) (layer B.Cu) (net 1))
 (segment (start 79.248 133.35) (end 79.248 130.302) (width 0.25) (layer B.Cu) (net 1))
 (segment (start 64.262 137.922) (end 64.339798 137.922) (width 0.25) (layer B.Cu) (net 1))
 (segment (start 64.339798 137.922) (end 64.410799 137.993001) (width 0.25) (layer B.Cu) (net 1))
 (segment (start 64.2278 137.922) (end 74.422 137.922) (width 0.25) (layer B.Cu) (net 1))
 (segment (start 64.169554 137.829554) (end 64.262 137.922) (width 0.25) (layer B.Cu) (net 1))
 (segment (start 64.169554 137.668) (end 64.169554 137.829554) (width 0.25) (layer B.Cu) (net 1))
 (segment (start 58.42 130.302) (end 58.42 131.918446) (width 0.25) (layer B.Cu) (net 1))
 (segment (start 58.42 131.918446) (end 64.169554 137.668) (width 0.25) (layer B.Cu) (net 1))
 (segment (start 74.422 120.396) (end 79.248 125.222) (width 0.25) (layer B.Cu) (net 1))
 (segment (start 79.248 125.222) (end 79.248 127.254) (width 0.25) (layer B.Cu) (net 1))
 (segment (start 73.152 120.396) (end 74.422 120.396) (width 0.25) (layer B.Cu) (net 1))
 (segment (start 72.136 119.38) (end 73.152 120.396) (width 0.25) (layer B.Cu) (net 1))
 (segment (start 72.136 117.856) (end 72.136 119.38) (width 0.25) (layer B.Cu) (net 1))
 (segment (start 78.74 111.252) (end 72.136 117.856) (width 0.25) (layer B.Cu) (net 1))
 (segment (start 78.74 102.333828) (end 78.74 111.252) (width 0.25) (layer B.Cu) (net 1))
 (segment (start 74.422 97.028) (end 74.422 98.015828) (width 0.25) (layer B.Cu) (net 1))
 (segment (start 74.422 98.015828) (end 78.74 102.333828) (width 0.25) (layer B.Cu) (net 1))
 (segment (start 79.248 127.254) (end 79.248 130.302) (width 0.25) (layer B.Cu) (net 1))
 (segment (start 58.42 127.254) (end 58.42 128.870446) (width 0.25) (layer B.Cu) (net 1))
 (segment (start 58.42 128.870446) (end 58.42 130.302) (width 0.25) (layer B.Cu) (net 1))
 (segment (start 64.262 117.094) (end 64.262 124.206) (width 0.25) (layer B.Cu) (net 2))
 (segment (start 64.262 124.206) (end 68.834 128.778) (width 0.25) (layer B.Cu) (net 2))
 (segment (start 61.976 114.808) (end 64.262 117.094) (width 0.25) (layer B.Cu) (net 2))
 (segment (start 61.976 114.554) (end 61.976 114.808) (width 0.25) (layer B.Cu) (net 2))
 (segment (start 56.896 109.474) (end 61.976 114.554) (width 0.25) (layer B.Cu) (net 2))
 (segment (start 56.896 97.028) (end 56.896 109.474) (width 0.25) (layer B.Cu) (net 2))
 (segment (start 67.056 98.552) (end 71.374 102.87) (width 0.25) (layer B.Cu) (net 3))
 (segment (start 71.374 102.87) (end 74.168 102.87) (width 0.25) (layer B.Cu) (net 3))
 (segment (start 67.056 97.028) (end 67.056 98.552) (width 0.25) (layer B.Cu) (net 3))
 (segment (start 63.112 100.076) (end 64.008 100.076) (width 0.25) (layer B.Cu) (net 3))
 (segment (start 64.008 100.076) (end 67.056 97.028) (width 0.25) (layer B.Cu) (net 3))
 (segment (start 61.214 103.124) (end 61.214 101.974) (width 0.25) (layer B.Cu) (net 3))
 (segment (start 61.214 101.974) (end 63.112 100.076) (width 0.25) (layer B.Cu) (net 3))
 (segment (start 61.214 105.664) (end 73.914 105.664) (width 0.25) (layer B.Cu) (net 4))
 (segment (start 73.914 105.664) (end 74.168 105.41) (width 0.25) (layer B.Cu) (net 4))
 (segment (start 71.882 97.028) (end 71.882 98.198998) (width 0.25) (layer B.Cu) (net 4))
 (segment (start 75.393001 104.184999) (end 75.067999 104.510001) (width 0.25) (layer B.Cu) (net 4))
 (segment (start 71.882 98.198998) (end 75.393001 101.709999) (width 0.25) (layer B.Cu) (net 4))
 (segment (start 75.393001 101.709999) (end 75.393001 104.184999) (width 0.25) (layer B.Cu) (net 4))
 (segment (start 75.067999 104.510001) (end 74.168 105.41) (width 0.25) (layer B.Cu) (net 4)))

